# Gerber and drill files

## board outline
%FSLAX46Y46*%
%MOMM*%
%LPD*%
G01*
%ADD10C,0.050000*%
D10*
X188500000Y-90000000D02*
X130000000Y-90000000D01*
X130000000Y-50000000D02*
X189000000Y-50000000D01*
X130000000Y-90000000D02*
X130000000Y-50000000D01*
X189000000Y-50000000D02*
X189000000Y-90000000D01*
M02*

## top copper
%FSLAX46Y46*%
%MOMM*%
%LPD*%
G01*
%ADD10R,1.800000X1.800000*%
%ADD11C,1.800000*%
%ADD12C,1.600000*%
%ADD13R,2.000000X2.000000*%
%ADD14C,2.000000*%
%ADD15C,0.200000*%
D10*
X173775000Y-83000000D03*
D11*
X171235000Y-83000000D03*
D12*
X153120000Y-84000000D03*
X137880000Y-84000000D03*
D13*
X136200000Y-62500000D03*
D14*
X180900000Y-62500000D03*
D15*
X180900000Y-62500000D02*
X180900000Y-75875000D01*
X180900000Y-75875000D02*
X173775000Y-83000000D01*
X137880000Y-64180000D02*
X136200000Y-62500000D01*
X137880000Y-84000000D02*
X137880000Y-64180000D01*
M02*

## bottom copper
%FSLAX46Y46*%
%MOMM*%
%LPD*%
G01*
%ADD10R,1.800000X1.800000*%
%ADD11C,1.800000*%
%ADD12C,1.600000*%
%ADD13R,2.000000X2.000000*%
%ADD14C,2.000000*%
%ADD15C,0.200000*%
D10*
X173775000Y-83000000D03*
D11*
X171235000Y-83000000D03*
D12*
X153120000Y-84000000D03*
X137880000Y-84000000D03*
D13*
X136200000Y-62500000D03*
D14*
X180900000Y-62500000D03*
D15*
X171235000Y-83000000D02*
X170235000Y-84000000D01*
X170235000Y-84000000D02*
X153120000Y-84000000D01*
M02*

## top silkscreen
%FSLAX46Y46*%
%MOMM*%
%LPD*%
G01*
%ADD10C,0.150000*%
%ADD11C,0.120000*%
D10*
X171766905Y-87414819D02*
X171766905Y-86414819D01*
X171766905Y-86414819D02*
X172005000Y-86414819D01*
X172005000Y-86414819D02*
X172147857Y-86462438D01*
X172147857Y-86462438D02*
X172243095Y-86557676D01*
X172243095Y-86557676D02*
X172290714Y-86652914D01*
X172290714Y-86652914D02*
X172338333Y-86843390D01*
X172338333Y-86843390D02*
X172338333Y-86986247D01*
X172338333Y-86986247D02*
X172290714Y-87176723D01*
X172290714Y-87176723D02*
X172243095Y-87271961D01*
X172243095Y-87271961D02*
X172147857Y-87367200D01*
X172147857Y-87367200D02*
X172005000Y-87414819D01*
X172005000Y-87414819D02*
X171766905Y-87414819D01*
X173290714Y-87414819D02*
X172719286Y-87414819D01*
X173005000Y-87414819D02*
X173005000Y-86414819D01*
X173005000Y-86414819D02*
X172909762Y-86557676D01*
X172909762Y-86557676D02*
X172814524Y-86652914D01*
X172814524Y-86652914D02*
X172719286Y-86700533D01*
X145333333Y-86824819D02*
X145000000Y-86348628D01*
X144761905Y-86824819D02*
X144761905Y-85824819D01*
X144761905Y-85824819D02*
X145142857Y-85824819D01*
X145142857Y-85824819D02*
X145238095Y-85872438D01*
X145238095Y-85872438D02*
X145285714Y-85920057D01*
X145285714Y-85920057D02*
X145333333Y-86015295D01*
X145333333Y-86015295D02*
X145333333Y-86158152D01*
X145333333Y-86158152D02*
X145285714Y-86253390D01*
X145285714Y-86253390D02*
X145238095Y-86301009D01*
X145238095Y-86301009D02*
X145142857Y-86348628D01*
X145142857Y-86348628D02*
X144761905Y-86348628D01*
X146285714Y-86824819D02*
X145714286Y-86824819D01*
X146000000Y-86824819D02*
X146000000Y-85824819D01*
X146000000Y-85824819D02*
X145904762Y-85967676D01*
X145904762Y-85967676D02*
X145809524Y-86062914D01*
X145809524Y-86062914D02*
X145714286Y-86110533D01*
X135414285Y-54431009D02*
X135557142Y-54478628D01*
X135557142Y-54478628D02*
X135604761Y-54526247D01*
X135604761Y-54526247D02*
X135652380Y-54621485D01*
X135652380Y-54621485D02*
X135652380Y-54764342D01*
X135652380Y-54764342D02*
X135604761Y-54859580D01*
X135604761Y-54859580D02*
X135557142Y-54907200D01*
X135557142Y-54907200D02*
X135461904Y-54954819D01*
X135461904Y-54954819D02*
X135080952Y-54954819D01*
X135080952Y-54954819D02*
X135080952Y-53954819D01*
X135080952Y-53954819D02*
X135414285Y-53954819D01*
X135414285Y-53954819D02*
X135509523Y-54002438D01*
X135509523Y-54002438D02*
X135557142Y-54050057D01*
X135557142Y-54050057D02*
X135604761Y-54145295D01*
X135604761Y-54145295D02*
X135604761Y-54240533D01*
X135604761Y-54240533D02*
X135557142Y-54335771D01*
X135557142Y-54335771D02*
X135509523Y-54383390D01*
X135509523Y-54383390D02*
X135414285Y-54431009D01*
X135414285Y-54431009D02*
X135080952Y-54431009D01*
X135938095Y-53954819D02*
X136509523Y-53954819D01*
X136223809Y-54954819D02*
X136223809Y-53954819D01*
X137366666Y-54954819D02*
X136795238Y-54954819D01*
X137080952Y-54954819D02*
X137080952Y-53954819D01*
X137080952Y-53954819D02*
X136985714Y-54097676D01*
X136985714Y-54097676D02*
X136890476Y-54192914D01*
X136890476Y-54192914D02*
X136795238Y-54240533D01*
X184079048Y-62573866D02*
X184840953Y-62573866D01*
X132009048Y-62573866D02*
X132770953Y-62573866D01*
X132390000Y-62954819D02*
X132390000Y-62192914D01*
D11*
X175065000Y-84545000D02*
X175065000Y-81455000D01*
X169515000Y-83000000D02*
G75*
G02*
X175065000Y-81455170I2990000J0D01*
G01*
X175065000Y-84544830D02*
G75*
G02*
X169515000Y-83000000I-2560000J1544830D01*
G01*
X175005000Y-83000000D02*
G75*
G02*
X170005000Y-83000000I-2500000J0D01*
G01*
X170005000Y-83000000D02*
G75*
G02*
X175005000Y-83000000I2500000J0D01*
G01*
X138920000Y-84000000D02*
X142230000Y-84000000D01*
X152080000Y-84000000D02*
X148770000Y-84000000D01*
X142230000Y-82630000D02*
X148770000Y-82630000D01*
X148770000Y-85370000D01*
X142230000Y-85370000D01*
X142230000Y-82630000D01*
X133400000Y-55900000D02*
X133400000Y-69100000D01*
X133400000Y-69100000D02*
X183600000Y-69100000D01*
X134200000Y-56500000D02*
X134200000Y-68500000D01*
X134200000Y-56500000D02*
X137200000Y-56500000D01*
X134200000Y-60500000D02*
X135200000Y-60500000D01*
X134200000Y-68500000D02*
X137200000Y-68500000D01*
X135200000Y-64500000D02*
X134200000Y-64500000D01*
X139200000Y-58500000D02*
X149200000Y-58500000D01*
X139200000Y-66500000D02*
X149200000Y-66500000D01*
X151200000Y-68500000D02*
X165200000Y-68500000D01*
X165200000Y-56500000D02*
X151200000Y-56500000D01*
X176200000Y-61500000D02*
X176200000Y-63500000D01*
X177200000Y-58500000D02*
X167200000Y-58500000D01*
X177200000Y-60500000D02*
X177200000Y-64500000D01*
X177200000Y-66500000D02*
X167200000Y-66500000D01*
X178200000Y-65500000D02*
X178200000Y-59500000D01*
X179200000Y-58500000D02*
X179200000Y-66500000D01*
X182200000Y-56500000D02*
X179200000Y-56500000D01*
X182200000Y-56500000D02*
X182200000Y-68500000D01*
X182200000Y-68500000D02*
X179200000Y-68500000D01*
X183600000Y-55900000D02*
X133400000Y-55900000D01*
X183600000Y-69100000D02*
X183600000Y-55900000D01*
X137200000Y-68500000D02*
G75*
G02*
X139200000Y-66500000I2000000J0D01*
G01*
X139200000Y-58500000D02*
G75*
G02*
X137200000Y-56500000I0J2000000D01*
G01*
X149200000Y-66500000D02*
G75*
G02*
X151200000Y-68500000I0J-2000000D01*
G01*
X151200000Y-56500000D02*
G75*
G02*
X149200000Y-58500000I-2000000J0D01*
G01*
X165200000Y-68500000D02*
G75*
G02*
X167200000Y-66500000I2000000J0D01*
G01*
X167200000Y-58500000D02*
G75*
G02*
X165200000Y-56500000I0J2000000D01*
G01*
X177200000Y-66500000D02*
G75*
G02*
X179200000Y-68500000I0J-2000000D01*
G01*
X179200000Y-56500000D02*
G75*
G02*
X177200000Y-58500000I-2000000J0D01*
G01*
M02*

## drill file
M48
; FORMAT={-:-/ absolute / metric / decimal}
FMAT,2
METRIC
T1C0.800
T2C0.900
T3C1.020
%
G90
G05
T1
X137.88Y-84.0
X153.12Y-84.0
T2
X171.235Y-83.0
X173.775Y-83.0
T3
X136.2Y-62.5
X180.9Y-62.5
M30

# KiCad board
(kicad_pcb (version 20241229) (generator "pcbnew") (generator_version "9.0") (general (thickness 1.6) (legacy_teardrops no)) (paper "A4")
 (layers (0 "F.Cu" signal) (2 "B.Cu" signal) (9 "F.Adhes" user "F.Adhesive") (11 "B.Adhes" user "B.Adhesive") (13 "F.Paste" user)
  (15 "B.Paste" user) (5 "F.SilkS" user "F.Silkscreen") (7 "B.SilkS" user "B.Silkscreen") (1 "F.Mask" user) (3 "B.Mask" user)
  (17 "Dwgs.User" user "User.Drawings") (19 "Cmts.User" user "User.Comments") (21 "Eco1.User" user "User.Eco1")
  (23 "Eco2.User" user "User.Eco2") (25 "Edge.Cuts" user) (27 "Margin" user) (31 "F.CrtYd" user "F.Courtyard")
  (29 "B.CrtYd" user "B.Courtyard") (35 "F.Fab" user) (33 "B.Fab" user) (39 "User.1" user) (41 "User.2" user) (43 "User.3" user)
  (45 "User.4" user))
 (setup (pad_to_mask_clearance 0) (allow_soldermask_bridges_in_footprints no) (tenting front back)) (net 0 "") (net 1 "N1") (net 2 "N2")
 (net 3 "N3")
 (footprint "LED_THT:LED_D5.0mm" (layer "F.Cu") (at 173.775 83 180)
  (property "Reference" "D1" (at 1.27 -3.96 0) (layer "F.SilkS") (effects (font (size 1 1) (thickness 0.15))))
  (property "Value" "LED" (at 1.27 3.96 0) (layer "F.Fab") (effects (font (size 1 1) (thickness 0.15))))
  (fp_line (start -1.29 -1.545) (end -1.29 1.545) (stroke (width 0.12) (type solid)) (layer "F.SilkS"))
  (fp_arc (start 4.26 0) (mid 2.071779 2.880495) (end -1.29 1.54483) (stroke (width 0.12) (type solid)) (layer "F.SilkS"))
  (fp_arc (start -1.29 -1.54483) (mid 2.071779 -2.880495) (end 4.26 0) (stroke (width 0.12) (type solid)) (layer "F.SilkS"))
  (fp_circle (center 1.27 0) (end 3.77 0) (stroke (width 0.12) (type solid)) (fill no) (layer "F.SilkS"))
  (pad "1" thru_hole rect (at 0 0 180) (size 1.8 1.8) (drill 0.9) (layers "*.Cu" "*.Mask") (remove_unused_layers no) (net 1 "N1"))
  (pad "2" thru_hole circle (at 2.54 0 180) (size 1.8 1.8) (drill 0.9) (layers "*.Cu" "*.Mask") (remove_unused_layers no) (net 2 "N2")))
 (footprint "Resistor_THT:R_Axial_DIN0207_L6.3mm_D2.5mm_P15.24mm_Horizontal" (layer "F.Cu") (at 153.12 84 180)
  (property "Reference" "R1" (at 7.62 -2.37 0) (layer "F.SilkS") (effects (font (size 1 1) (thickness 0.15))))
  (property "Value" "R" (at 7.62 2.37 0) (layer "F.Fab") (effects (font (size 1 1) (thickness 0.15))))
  (fp_line (start 14.2 0) (end 10.89 0) (stroke (width 0.12) (type solid)) (layer "F.SilkS"))
  (fp_line (start 1.04 0) (end 4.35 0) (stroke (width 0.12) (type solid)) (layer "F.SilkS"))
  (fp_rect (start 4.35 -1.37) (end 10.89 1.37) (stroke (width 0.12) (type solid)) (fill no) (layer "F.SilkS"))
  (pad "1" thru_hole circle (at 0 0 180) (size 1.6 1.6) (drill 0.8) (layers "*.Cu" "*.Mask") (remove_unused_layers no) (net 2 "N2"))
  (pad "2" thru_hole circle (at 15.24 0 180) (size 1.6 1.6) (drill 0.8) (layers "*.Cu" "*.Mask") (remove_unused_layers no) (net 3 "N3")))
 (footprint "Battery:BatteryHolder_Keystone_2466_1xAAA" (layer "F.Cu") (at 136.2 62.5)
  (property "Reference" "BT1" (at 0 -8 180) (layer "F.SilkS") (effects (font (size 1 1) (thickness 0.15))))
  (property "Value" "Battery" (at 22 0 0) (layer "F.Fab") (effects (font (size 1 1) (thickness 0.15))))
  (fp_line (start -2.8 -6.6) (end -2.8 6.6) (stroke (width 0.12) (type solid)) (layer "F.SilkS"))
  (fp_line (start -2.8 6.6) (end 47.4 6.6) (stroke (width 0.12) (type solid)) (layer "F.SilkS"))
  (fp_line (start -2 -6) (end -2 6) (stroke (width 0.12) (type solid)) (layer "F.SilkS"))
  (fp_line (start -2 -6) (end 1 -6) (stroke (width 0.12) (type solid)) (layer "F.SilkS"))
  (fp_line (start -2 -2) (end -1 -2) (stroke (width 0.12) (type solid)) (layer "F.SilkS"))
  (fp_line (start -2 6) (end 1 6) (stroke (width 0.12) (type solid)) (layer "F.SilkS"))
  (fp_line (start -1 2) (end -2 2) (stroke (width 0.12) (type solid)) (layer "F.SilkS"))
  (fp_line (start 3 -4) (end 13 -4) (stroke (width 0.12) (type solid)) (layer "F.SilkS"))
  (fp_line (start 3 4) (end 13 4) (stroke (width 0.12) (type solid)) (layer "F.SilkS"))
  (fp_line (start 15 6) (end 29 6) (stroke (width 0.12) (type solid)) (layer "F.SilkS"))
  (fp_line (start 29 -6) (end 15 -6) (stroke (width 0.12) (type solid)) (layer "F.SilkS"))
  (fp_line (start 40 -1) (end 40 1) (stroke (width 0.12) (type solid)) (layer "F.SilkS"))
  (fp_line (start 41 -4) (end 31 -4) (stroke (width 0.12) (type solid)) (layer "F.SilkS"))
  (fp_line (start 41 -2) (end 41 2) (stroke (width 0.12) (type solid)) (layer "F.SilkS"))
  (fp_line (start 41 4) (end 31 4) (stroke (width 0.12) (type solid)) (layer "F.SilkS"))
  (fp_line (start 42 3) (end 42 -3) (stroke (width 0.12) (type solid)) (layer "F.SilkS"))
  (fp_line (start 43 -4) (end 43 4) (stroke (width 0.12) (type solid)) (layer "F.SilkS"))
  (fp_line (start 46 -6) (end 43 -6) (stroke (width 0.12) (type solid)) (layer "F.SilkS"))
  (fp_line (start 46 -6) (end 46 6) (stroke (width 0.12) (type solid)) (layer "F.SilkS"))
  (fp_line (start 46 6) (end 43 6) (stroke (width 0.12) (type solid)) (layer "F.SilkS"))
  (fp_line (start 47.4 -6.6) (end -2.8 -6.6) (stroke (width 0.12) (type solid)) (layer "F.SilkS"))
  (fp_line (start 47.4 6.6) (end 47.4 -6.6) (stroke (width 0.12) (type solid)) (layer "F.SilkS"))
  (fp_arc (start 1 6) (mid 1.585786 4.585786) (end 3 4) (stroke (width 0.12) (type solid)) (layer "F.SilkS"))
  (fp_arc (start 3 -4) (mid 1.585786 -4.585786) (end 1 -6) (stroke (width 0.12) (type solid)) (layer "F.SilkS"))
  (fp_arc (start 13 4) (mid 14.414214 4.585786) (end 15 6) (stroke (width 0.12) (type solid)) (layer "F.SilkS"))
  (fp_arc (start 15 -6) (mid 14.414214 -4.585786) (end 13 -4) (stroke (width 0.12) (type solid)) (layer "F.SilkS"))
  (fp_arc (start 29 6) (mid 29.585786 4.585786) (end 31 4) (stroke (width 0.12) (type solid)) (layer "F.SilkS"))
  (fp_arc (start 31 -4) (mid 29.585786 -4.585786) (end 29 -6) (stroke (width 0.12) (type solid)) (layer "F.SilkS"))
  (fp_arc (start 41 4) (mid 42.414214 4.585786) (end 43 6) (stroke (width 0.12) (type solid)) (layer "F.SilkS"))
  (fp_arc (start 43 -6) (mid 42.414214 -4.585786) (end 41 -4) (stroke (width 0.12) (type solid)) (layer "F.SilkS"))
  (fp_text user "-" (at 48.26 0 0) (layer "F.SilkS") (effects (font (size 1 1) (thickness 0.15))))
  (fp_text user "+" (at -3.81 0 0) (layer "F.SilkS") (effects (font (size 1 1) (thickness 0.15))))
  (pad "1" thru_hole rect (at 0 0) (size 2 2) (drill 1.02) (layers "*.Cu" "*.Mask") (remove_unused_layers no) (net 3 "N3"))
  (pad "2" thru_hole circle (at 44.7 0) (size 2 2) (drill 1.02) (layers "*.Cu" "*.Mask") (remove_unused_layers no) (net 1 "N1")))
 (gr_line (start 188.5 90) (end 130 90) (stroke (width 0.05) (type default)) (layer "Edge.Cuts"))
 (gr_line (start 130 50) (end 189 50) (stroke (width 0.05) (type default)) (layer "Edge.Cuts"))
 (gr_line (start 130 90) (end 130 50) (stroke (width 0.05) (type default)) (layer "Edge.Cuts"))
 (gr_line (start 189 50) (end 189 90) (stroke (width 0.05) (type default)) (layer "Edge.Cuts"))
 (segment (start 180.9 62.5) (end 180.9 75.875) (width 0.2) (layer "F.Cu") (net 1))
 (segment (start 180.9 75.875) (end 173.775 83) (width 0.2) (layer "F.Cu") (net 1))
 (segment (start 137.88 64.18) (end 136.2 62.5) (width 0.2) (layer "F.Cu") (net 3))
 (segment (start 137.88 84) (end 137.88 64.18) (width 0.2) (layer "F.Cu") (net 3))
 (segment (start 171.235 83) (end 170.235 84) (width 0.2) (layer "B.Cu") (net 2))
 (segment (start 170.235 84) (end 153.12 84) (width 0.2) (layer "B.Cu") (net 2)))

